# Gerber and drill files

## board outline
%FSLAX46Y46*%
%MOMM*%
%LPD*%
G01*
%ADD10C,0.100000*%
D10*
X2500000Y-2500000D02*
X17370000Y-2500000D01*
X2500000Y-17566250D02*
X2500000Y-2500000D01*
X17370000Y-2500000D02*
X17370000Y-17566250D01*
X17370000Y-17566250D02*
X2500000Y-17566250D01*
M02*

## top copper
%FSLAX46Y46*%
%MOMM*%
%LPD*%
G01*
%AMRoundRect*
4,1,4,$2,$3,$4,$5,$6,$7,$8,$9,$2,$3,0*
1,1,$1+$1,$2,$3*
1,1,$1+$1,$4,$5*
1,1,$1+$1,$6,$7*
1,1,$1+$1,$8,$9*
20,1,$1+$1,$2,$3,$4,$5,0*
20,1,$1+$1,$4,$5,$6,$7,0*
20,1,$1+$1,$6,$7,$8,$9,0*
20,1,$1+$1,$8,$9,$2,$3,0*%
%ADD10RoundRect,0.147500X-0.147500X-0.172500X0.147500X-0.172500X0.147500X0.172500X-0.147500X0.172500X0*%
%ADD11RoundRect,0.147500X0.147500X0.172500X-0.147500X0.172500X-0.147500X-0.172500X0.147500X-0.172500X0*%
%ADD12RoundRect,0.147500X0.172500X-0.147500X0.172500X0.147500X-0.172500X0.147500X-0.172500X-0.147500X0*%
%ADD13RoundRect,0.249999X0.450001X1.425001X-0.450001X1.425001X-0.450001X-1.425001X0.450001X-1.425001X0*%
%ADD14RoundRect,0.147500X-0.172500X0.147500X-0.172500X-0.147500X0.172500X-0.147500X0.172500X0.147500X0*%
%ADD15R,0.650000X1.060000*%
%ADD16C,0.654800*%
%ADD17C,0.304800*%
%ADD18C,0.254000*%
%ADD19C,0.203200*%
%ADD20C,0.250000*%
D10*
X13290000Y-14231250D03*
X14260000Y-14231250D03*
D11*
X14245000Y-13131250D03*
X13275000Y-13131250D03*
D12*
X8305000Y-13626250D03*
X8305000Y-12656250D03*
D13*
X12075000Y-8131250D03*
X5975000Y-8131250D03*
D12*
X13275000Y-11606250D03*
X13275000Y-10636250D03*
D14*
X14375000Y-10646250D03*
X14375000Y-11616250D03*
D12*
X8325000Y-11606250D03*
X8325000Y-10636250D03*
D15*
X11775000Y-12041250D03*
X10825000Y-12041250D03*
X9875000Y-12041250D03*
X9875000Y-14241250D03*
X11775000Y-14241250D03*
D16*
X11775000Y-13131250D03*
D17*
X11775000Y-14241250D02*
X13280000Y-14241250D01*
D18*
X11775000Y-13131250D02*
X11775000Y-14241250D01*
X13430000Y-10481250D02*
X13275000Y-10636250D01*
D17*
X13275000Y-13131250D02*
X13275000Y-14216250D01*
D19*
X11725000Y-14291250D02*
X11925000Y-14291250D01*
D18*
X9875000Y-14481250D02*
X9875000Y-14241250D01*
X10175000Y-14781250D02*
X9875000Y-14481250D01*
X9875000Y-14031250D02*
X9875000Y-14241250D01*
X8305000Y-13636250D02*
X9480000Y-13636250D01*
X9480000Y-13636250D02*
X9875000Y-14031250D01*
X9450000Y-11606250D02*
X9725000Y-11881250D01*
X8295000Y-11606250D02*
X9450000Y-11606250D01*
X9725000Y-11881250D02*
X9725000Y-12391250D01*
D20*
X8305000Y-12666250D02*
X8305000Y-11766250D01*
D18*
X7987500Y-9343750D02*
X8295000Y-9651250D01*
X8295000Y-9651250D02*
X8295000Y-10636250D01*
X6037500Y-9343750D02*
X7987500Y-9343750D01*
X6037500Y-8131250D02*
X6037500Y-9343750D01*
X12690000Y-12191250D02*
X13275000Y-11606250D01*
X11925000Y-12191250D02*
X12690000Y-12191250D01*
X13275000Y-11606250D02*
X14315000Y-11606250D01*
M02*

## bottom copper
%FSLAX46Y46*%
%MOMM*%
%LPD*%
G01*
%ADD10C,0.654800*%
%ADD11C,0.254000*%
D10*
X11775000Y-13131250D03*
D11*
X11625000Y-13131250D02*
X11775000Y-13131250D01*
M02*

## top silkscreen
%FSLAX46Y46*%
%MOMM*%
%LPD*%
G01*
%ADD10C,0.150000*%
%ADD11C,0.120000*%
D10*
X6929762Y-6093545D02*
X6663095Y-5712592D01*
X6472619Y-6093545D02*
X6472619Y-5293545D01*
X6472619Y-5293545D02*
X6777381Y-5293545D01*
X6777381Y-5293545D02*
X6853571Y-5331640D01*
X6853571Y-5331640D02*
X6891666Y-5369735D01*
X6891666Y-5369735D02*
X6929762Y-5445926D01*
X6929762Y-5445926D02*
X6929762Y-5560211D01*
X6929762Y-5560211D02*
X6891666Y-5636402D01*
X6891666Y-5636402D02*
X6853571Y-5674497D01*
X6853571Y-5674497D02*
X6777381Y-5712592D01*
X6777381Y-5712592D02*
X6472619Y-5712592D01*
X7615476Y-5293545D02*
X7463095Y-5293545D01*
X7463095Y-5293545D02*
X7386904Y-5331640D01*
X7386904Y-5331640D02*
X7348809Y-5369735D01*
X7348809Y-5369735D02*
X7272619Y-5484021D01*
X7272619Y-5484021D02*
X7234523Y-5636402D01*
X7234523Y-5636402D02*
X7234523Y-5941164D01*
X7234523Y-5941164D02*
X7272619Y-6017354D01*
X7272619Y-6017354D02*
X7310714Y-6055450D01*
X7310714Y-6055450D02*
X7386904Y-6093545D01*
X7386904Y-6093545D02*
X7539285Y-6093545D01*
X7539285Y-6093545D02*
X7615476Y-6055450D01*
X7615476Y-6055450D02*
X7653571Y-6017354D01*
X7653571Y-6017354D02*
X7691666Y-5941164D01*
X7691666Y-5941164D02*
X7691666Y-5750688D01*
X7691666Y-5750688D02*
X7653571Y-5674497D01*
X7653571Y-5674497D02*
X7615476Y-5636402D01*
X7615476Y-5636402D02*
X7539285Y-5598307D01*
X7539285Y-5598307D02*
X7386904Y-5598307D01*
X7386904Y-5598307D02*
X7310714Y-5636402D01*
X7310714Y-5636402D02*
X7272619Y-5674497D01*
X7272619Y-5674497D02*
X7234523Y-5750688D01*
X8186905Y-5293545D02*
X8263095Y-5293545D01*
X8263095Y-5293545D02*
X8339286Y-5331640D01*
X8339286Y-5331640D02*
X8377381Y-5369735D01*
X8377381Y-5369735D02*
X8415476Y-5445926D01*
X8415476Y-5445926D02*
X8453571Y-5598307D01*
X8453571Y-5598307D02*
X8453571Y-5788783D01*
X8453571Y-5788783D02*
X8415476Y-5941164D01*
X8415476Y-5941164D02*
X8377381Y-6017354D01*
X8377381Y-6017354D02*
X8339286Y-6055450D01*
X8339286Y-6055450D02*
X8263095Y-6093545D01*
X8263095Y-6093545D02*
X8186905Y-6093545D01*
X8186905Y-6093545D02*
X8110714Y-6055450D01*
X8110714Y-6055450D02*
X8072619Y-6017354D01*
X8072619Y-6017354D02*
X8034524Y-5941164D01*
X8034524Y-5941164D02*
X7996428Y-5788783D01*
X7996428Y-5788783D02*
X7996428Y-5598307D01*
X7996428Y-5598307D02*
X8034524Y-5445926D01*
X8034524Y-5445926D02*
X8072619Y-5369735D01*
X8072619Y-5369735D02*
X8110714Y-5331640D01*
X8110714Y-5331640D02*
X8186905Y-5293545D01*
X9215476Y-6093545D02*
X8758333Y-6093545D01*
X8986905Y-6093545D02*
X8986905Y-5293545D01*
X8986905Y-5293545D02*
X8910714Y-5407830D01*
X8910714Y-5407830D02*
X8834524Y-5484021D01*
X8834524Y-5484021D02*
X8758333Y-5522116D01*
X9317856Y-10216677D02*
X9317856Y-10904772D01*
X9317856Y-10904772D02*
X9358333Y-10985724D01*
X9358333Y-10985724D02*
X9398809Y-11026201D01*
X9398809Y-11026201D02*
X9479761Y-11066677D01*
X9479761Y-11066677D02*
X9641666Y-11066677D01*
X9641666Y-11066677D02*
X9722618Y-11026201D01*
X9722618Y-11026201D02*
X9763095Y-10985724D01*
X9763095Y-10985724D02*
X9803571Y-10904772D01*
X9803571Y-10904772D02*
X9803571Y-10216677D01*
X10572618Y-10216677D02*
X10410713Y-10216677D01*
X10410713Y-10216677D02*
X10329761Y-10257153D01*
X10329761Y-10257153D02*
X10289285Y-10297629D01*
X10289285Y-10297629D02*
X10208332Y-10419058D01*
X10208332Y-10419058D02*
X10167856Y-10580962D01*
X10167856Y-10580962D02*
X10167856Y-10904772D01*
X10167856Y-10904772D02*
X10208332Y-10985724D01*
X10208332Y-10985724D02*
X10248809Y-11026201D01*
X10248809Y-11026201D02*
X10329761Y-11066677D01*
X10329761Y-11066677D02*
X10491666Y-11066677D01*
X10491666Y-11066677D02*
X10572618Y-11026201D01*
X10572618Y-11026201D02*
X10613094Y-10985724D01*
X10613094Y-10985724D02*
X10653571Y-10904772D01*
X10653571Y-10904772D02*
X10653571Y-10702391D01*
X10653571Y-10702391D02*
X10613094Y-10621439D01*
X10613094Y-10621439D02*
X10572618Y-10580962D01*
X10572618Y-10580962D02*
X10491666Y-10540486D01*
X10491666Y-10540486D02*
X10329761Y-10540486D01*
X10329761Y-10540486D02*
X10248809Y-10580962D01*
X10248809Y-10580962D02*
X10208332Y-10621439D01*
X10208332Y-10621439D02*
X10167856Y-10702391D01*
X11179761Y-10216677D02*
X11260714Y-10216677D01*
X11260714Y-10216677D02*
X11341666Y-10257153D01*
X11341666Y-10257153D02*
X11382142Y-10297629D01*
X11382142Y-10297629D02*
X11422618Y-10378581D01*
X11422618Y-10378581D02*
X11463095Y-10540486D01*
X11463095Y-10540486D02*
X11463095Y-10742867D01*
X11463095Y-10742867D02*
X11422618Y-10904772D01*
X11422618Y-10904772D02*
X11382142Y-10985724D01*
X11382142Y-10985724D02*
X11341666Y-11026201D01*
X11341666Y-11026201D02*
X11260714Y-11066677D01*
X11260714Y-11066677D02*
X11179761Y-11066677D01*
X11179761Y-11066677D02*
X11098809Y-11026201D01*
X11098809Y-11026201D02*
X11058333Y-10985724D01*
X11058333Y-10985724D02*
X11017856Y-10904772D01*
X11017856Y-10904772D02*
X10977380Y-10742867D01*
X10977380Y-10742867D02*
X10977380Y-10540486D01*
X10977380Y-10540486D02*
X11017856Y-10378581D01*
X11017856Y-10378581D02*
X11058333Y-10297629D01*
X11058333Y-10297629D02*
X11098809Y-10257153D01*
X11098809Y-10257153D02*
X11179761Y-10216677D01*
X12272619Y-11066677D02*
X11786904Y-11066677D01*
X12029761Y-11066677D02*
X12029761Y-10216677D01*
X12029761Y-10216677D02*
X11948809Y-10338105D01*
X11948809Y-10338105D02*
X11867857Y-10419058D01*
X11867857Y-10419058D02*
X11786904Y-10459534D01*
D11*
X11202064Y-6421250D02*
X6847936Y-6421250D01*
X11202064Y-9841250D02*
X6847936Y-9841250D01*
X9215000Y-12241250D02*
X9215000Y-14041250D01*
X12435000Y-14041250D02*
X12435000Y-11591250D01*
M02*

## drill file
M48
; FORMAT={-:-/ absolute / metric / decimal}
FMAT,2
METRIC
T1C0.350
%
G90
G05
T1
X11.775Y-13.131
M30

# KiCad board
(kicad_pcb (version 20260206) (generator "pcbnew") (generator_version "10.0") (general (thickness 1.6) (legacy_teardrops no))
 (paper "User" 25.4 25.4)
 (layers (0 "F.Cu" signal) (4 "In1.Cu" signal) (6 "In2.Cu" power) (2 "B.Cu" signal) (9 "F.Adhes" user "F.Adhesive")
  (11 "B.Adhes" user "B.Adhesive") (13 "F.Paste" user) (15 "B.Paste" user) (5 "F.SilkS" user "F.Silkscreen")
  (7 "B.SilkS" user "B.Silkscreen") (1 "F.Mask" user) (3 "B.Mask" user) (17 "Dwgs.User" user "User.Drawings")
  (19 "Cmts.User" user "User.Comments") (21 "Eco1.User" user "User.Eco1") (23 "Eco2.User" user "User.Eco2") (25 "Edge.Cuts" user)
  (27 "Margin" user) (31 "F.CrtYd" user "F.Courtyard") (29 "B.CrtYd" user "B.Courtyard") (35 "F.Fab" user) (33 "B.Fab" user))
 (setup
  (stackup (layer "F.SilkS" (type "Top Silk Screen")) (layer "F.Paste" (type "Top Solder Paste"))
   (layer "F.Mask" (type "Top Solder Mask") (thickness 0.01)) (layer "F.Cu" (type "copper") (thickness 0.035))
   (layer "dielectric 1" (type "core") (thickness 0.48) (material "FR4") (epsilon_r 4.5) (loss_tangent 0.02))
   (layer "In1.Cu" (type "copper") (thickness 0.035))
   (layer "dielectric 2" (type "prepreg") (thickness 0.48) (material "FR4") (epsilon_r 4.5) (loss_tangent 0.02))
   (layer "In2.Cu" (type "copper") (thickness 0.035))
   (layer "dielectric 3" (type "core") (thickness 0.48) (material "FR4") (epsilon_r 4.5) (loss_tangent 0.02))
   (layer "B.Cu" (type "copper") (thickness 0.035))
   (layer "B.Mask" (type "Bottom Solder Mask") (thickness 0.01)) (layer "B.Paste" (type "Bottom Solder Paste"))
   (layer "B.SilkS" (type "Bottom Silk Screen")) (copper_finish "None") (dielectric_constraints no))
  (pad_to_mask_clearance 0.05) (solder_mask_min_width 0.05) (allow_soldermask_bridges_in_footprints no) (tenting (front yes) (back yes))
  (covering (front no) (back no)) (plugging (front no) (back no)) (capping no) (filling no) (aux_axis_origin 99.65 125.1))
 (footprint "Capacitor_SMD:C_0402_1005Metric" (layer "F.Cu") (at 13.775 14.23125)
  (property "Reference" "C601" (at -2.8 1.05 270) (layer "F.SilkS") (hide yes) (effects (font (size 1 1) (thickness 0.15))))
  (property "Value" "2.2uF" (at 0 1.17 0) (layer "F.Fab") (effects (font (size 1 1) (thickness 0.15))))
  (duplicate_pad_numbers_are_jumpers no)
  (pad "1" smd roundrect (at -0.485 0) (size 0.59 0.64) (layers "F.Cu" "F.Mask" "F.Paste") (roundrect_rratio 0.25) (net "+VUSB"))
  (pad "2" smd roundrect (at 0.485 0) (size 0.59 0.64) (layers "F.Cu" "F.Mask" "F.Paste") (roundrect_rratio 0.25) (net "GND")))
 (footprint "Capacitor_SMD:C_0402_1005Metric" (layer "F.Cu") (at 13.76 13.13125 180)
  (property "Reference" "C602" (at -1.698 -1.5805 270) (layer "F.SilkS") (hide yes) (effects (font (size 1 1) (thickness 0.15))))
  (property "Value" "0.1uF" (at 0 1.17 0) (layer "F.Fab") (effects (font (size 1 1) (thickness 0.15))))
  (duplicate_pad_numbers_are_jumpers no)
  (pad "1" smd roundrect (at -0.485 0 180) (size 0.59 0.64) (layers "F.Cu" "F.Mask" "F.Paste") (roundrect_rratio 0.25) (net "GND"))
  (pad "2" smd roundrect (at 0.485 0 180) (size 0.59 0.64) (layers "F.Cu" "F.Mask" "F.Paste") (roundrect_rratio 0.25) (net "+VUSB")))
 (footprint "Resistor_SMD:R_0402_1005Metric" (layer "F.Cu") (at 8.305 13.14125 90)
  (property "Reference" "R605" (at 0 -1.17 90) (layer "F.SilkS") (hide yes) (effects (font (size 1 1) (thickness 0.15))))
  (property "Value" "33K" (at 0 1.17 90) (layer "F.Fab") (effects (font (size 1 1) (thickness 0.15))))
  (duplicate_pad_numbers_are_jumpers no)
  (pad "1" smd roundrect (at -0.485 0 90) (size 0.59 0.64) (layers "F.Cu" "F.Mask" "F.Paste") (roundrect_rratio 0.25) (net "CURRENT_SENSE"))
  (pad "2" smd roundrect (at 0.485 0 90) (size 0.59 0.64) (layers "F.Cu" "F.Mask" "F.Paste") (roundrect_rratio 0.25) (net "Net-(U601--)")))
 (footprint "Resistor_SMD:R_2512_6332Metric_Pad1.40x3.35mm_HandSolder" (layer "F.Cu") (at 9.025 8.13125 180)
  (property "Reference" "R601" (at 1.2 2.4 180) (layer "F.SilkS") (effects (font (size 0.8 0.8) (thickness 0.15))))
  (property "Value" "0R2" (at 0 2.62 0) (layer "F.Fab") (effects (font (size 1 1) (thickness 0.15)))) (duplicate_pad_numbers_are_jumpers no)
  (fp_line (start -2.177064 1.71) (end 2.177064 1.71) (stroke (width 0.12) (type solid)) (layer "F.SilkS"))
  (fp_line (start -2.177064 -1.71) (end 2.177064 -1.71) (stroke (width 0.12) (type solid)) (layer "F.SilkS"))
  (pad "1" smd roundrect (at -3.05 0 180) (size 1.4 3.35) (layers "F.Cu" "F.Mask" "F.Paste") (roundrect_rratio 0.1785707143) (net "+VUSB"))
  (pad "2" smd roundrect (at 3.05 0 180) (size 1.4 3.35) (layers "F.Cu" "F.Mask" "F.Paste") (roundrect_rratio 0.1785707143) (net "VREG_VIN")))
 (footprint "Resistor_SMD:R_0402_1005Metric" (layer "F.Cu") (at 13.275 11.12125 90)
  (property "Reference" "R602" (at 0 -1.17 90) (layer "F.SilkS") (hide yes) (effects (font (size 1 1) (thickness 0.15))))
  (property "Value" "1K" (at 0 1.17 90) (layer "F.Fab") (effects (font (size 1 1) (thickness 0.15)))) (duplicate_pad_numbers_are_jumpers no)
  (pad "1" smd roundrect (at -0.485 0 90) (size 0.59 0.64) (layers "F.Cu" "F.Mask" "F.Paste") (roundrect_rratio 0.25) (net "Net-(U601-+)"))
  (pad "2" smd roundrect (at 0.485 0 90) (size 0.59 0.64) (layers "F.Cu" "F.Mask" "F.Paste") (roundrect_rratio 0.25) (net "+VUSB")))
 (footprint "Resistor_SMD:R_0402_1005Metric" (layer "F.Cu") (at 14.375 11.13125 -90)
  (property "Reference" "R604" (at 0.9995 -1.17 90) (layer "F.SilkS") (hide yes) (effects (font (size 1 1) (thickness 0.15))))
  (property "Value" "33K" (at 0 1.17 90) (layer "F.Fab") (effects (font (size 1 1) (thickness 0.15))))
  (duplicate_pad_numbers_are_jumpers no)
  (pad "1" smd roundrect (at -0.485 0 270) (size 0.59 0.64) (layers "F.Cu" "F.Mask" "F.Paste") (roundrect_rratio 0.25) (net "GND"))
  (pad "2" smd roundrect (at 0.485 0 270) (size 0.59 0.64) (layers "F.Cu" "F.Mask" "F.Paste") (roundrect_rratio 0.25) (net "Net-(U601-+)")))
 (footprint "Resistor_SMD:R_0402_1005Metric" (layer "F.Cu") (at 8.325 11.12125 90)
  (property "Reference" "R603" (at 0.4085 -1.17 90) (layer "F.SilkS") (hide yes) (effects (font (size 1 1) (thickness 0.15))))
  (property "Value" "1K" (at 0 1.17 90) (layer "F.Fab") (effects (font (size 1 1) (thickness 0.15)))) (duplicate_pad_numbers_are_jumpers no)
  (pad "1" smd roundrect (at -0.485 0 90) (size 0.59 0.64) (layers "F.Cu" "F.Mask" "F.Paste") (roundrect_rratio 0.25) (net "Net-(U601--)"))
  (pad "2" smd roundrect (at 0.485 0 90) (size 0.59 0.64) (layers "F.Cu" "F.Mask" "F.Paste") (roundrect_rratio 0.25) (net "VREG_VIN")))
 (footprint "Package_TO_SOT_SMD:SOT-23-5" (layer "F.Cu") (at 10.825 13.14125 -90)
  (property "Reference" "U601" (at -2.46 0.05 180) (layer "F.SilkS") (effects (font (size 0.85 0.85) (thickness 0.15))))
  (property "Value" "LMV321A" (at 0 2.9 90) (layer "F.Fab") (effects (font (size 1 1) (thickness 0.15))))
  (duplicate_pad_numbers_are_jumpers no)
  (fp_line (start -0.9 1.61) (end 0.9 1.61) (stroke (width 0.12) (type solid)) (layer "F.SilkS"))
  (fp_line (start 0.9 -1.61) (end -1.55 -1.61) (stroke (width 0.12) (type solid)) (layer "F.SilkS"))
  (pad "1" smd rect (at -1.1 -0.95 270) (size 1.06 0.65) (layers "F.Cu" "F.Mask" "F.Paste") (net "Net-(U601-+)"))
  (pad "2" smd rect (at -1.1 0 270) (size 1.06 0.65) (layers "F.Cu" "F.Mask" "F.Paste") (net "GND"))
  (pad "3" smd rect (at -1.1 0.95 270) (size 1.06 0.65) (layers "F.Cu" "F.Mask" "F.Paste") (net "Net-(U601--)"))
  (pad "4" smd rect (at 1.1 0.95 270) (size 1.06 0.65) (layers "F.Cu" "F.Mask" "F.Paste") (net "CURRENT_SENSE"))
  (pad "5" smd rect (at 1.1 -0.95 270) (size 1.06 0.65) (layers "F.Cu" "F.Mask" "F.Paste") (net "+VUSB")))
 (gr_line (start 2.5 2.5) (end 17.37 2.5) (stroke (width 0.1) (type default)) (layer "Edge.Cuts"))
 (gr_line (start 2.5 17.56625) (end 2.5 2.5) (stroke (width 0.1) (type default)) (layer "Edge.Cuts"))
 (gr_line (start 17.37 2.5) (end 17.37 17.56625) (stroke (width 0.1) (type default)) (layer "Edge.Cuts"))
 (gr_line (start 17.37 17.56625) (end 2.5 17.56625) (stroke (width 0.1) (type default)) (layer "Edge.Cuts"))
 (segment (start 11.775 14.24125) (end 13.28 14.24125) (width 0.3048) (layer "F.Cu") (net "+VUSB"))
 (segment (start 11.775 13.13125) (end 11.775 14.24125) (width 0.254) (layer "F.Cu") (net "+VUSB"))
 (segment (start 13.43 10.48125) (end 13.275 10.63625) (width 0.254) (layer "F.Cu") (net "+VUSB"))
 (segment (start 13.275 13.13125) (end 13.275 14.21625) (width 0.3048) (layer "F.Cu") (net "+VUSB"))
 (segment (start 11.725 14.29125) (end 11.925 14.29125) (width 0.2032) (layer "F.Cu") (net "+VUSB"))
 (via (at 11.775 13.13125) (size 0.6548) (drill 0.35) (layers "F.Cu" "B.Cu") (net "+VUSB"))
 (segment (start 11.625 13.13125) (end 11.775 13.13125) (width 0.254) (layer "B.Cu") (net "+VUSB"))
 (segment (start 9.875 14.48125) (end 9.875 14.24125) (width 0.254) (layer "F.Cu") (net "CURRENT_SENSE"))
 (segment (start 10.175 14.78125) (end 9.875 14.48125) (width 0.254) (layer "F.Cu") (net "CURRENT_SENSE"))
 (segment (start 9.875 14.03125) (end 9.875 14.24125) (width 0.254) (layer "F.Cu") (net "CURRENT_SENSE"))
 (segment (start 8.305 13.63625) (end 9.48 13.63625) (width 0.254) (layer "F.Cu") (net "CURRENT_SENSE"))
 (segment (start 9.48 13.63625) (end 9.875 14.03125) (width 0.254) (layer "F.Cu") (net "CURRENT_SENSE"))
 (segment (start 9.45 11.60625) (end 9.725 11.88125) (width 0.254) (layer "F.Cu") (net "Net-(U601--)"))
 (segment (start 8.295 11.60625) (end 9.45 11.60625) (width 0.254) (layer "F.Cu") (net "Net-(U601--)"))
 (segment (start 9.725 11.88125) (end 9.725 12.39125) (width 0.254) (layer "F.Cu") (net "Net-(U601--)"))
 (segment (start 8.305 12.66625) (end 8.305 11.76625) (width 0.25) (layer "F.Cu") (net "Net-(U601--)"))
 (segment (start 7.9875 9.34375) (end 8.295 9.65125) (width 0.254) (layer "F.Cu") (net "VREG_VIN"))
 (segment (start 8.295 9.65125) (end 8.295 10.63625) (width 0.254) (layer "F.Cu") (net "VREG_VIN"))
 (segment (start 6.0375 9.34375) (end 7.9875 9.34375) (width 0.254) (layer "F.Cu") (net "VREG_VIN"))
 (segment (start 6.0375 8.13125) (end 6.0375 9.34375) (width 0.254) (layer "F.Cu") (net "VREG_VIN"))
 (segment (start 12.69 12.19125) (end 13.275 11.60625) (width 0.254) (layer "F.Cu") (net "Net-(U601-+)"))
 (segment (start 11.925 12.19125) (end 12.69 12.19125) (width 0.254) (layer "F.Cu") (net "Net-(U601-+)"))
 (segment (start 13.275 11.60625) (end 14.315 11.60625) (width 0.254) (layer "F.Cu") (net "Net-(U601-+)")))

